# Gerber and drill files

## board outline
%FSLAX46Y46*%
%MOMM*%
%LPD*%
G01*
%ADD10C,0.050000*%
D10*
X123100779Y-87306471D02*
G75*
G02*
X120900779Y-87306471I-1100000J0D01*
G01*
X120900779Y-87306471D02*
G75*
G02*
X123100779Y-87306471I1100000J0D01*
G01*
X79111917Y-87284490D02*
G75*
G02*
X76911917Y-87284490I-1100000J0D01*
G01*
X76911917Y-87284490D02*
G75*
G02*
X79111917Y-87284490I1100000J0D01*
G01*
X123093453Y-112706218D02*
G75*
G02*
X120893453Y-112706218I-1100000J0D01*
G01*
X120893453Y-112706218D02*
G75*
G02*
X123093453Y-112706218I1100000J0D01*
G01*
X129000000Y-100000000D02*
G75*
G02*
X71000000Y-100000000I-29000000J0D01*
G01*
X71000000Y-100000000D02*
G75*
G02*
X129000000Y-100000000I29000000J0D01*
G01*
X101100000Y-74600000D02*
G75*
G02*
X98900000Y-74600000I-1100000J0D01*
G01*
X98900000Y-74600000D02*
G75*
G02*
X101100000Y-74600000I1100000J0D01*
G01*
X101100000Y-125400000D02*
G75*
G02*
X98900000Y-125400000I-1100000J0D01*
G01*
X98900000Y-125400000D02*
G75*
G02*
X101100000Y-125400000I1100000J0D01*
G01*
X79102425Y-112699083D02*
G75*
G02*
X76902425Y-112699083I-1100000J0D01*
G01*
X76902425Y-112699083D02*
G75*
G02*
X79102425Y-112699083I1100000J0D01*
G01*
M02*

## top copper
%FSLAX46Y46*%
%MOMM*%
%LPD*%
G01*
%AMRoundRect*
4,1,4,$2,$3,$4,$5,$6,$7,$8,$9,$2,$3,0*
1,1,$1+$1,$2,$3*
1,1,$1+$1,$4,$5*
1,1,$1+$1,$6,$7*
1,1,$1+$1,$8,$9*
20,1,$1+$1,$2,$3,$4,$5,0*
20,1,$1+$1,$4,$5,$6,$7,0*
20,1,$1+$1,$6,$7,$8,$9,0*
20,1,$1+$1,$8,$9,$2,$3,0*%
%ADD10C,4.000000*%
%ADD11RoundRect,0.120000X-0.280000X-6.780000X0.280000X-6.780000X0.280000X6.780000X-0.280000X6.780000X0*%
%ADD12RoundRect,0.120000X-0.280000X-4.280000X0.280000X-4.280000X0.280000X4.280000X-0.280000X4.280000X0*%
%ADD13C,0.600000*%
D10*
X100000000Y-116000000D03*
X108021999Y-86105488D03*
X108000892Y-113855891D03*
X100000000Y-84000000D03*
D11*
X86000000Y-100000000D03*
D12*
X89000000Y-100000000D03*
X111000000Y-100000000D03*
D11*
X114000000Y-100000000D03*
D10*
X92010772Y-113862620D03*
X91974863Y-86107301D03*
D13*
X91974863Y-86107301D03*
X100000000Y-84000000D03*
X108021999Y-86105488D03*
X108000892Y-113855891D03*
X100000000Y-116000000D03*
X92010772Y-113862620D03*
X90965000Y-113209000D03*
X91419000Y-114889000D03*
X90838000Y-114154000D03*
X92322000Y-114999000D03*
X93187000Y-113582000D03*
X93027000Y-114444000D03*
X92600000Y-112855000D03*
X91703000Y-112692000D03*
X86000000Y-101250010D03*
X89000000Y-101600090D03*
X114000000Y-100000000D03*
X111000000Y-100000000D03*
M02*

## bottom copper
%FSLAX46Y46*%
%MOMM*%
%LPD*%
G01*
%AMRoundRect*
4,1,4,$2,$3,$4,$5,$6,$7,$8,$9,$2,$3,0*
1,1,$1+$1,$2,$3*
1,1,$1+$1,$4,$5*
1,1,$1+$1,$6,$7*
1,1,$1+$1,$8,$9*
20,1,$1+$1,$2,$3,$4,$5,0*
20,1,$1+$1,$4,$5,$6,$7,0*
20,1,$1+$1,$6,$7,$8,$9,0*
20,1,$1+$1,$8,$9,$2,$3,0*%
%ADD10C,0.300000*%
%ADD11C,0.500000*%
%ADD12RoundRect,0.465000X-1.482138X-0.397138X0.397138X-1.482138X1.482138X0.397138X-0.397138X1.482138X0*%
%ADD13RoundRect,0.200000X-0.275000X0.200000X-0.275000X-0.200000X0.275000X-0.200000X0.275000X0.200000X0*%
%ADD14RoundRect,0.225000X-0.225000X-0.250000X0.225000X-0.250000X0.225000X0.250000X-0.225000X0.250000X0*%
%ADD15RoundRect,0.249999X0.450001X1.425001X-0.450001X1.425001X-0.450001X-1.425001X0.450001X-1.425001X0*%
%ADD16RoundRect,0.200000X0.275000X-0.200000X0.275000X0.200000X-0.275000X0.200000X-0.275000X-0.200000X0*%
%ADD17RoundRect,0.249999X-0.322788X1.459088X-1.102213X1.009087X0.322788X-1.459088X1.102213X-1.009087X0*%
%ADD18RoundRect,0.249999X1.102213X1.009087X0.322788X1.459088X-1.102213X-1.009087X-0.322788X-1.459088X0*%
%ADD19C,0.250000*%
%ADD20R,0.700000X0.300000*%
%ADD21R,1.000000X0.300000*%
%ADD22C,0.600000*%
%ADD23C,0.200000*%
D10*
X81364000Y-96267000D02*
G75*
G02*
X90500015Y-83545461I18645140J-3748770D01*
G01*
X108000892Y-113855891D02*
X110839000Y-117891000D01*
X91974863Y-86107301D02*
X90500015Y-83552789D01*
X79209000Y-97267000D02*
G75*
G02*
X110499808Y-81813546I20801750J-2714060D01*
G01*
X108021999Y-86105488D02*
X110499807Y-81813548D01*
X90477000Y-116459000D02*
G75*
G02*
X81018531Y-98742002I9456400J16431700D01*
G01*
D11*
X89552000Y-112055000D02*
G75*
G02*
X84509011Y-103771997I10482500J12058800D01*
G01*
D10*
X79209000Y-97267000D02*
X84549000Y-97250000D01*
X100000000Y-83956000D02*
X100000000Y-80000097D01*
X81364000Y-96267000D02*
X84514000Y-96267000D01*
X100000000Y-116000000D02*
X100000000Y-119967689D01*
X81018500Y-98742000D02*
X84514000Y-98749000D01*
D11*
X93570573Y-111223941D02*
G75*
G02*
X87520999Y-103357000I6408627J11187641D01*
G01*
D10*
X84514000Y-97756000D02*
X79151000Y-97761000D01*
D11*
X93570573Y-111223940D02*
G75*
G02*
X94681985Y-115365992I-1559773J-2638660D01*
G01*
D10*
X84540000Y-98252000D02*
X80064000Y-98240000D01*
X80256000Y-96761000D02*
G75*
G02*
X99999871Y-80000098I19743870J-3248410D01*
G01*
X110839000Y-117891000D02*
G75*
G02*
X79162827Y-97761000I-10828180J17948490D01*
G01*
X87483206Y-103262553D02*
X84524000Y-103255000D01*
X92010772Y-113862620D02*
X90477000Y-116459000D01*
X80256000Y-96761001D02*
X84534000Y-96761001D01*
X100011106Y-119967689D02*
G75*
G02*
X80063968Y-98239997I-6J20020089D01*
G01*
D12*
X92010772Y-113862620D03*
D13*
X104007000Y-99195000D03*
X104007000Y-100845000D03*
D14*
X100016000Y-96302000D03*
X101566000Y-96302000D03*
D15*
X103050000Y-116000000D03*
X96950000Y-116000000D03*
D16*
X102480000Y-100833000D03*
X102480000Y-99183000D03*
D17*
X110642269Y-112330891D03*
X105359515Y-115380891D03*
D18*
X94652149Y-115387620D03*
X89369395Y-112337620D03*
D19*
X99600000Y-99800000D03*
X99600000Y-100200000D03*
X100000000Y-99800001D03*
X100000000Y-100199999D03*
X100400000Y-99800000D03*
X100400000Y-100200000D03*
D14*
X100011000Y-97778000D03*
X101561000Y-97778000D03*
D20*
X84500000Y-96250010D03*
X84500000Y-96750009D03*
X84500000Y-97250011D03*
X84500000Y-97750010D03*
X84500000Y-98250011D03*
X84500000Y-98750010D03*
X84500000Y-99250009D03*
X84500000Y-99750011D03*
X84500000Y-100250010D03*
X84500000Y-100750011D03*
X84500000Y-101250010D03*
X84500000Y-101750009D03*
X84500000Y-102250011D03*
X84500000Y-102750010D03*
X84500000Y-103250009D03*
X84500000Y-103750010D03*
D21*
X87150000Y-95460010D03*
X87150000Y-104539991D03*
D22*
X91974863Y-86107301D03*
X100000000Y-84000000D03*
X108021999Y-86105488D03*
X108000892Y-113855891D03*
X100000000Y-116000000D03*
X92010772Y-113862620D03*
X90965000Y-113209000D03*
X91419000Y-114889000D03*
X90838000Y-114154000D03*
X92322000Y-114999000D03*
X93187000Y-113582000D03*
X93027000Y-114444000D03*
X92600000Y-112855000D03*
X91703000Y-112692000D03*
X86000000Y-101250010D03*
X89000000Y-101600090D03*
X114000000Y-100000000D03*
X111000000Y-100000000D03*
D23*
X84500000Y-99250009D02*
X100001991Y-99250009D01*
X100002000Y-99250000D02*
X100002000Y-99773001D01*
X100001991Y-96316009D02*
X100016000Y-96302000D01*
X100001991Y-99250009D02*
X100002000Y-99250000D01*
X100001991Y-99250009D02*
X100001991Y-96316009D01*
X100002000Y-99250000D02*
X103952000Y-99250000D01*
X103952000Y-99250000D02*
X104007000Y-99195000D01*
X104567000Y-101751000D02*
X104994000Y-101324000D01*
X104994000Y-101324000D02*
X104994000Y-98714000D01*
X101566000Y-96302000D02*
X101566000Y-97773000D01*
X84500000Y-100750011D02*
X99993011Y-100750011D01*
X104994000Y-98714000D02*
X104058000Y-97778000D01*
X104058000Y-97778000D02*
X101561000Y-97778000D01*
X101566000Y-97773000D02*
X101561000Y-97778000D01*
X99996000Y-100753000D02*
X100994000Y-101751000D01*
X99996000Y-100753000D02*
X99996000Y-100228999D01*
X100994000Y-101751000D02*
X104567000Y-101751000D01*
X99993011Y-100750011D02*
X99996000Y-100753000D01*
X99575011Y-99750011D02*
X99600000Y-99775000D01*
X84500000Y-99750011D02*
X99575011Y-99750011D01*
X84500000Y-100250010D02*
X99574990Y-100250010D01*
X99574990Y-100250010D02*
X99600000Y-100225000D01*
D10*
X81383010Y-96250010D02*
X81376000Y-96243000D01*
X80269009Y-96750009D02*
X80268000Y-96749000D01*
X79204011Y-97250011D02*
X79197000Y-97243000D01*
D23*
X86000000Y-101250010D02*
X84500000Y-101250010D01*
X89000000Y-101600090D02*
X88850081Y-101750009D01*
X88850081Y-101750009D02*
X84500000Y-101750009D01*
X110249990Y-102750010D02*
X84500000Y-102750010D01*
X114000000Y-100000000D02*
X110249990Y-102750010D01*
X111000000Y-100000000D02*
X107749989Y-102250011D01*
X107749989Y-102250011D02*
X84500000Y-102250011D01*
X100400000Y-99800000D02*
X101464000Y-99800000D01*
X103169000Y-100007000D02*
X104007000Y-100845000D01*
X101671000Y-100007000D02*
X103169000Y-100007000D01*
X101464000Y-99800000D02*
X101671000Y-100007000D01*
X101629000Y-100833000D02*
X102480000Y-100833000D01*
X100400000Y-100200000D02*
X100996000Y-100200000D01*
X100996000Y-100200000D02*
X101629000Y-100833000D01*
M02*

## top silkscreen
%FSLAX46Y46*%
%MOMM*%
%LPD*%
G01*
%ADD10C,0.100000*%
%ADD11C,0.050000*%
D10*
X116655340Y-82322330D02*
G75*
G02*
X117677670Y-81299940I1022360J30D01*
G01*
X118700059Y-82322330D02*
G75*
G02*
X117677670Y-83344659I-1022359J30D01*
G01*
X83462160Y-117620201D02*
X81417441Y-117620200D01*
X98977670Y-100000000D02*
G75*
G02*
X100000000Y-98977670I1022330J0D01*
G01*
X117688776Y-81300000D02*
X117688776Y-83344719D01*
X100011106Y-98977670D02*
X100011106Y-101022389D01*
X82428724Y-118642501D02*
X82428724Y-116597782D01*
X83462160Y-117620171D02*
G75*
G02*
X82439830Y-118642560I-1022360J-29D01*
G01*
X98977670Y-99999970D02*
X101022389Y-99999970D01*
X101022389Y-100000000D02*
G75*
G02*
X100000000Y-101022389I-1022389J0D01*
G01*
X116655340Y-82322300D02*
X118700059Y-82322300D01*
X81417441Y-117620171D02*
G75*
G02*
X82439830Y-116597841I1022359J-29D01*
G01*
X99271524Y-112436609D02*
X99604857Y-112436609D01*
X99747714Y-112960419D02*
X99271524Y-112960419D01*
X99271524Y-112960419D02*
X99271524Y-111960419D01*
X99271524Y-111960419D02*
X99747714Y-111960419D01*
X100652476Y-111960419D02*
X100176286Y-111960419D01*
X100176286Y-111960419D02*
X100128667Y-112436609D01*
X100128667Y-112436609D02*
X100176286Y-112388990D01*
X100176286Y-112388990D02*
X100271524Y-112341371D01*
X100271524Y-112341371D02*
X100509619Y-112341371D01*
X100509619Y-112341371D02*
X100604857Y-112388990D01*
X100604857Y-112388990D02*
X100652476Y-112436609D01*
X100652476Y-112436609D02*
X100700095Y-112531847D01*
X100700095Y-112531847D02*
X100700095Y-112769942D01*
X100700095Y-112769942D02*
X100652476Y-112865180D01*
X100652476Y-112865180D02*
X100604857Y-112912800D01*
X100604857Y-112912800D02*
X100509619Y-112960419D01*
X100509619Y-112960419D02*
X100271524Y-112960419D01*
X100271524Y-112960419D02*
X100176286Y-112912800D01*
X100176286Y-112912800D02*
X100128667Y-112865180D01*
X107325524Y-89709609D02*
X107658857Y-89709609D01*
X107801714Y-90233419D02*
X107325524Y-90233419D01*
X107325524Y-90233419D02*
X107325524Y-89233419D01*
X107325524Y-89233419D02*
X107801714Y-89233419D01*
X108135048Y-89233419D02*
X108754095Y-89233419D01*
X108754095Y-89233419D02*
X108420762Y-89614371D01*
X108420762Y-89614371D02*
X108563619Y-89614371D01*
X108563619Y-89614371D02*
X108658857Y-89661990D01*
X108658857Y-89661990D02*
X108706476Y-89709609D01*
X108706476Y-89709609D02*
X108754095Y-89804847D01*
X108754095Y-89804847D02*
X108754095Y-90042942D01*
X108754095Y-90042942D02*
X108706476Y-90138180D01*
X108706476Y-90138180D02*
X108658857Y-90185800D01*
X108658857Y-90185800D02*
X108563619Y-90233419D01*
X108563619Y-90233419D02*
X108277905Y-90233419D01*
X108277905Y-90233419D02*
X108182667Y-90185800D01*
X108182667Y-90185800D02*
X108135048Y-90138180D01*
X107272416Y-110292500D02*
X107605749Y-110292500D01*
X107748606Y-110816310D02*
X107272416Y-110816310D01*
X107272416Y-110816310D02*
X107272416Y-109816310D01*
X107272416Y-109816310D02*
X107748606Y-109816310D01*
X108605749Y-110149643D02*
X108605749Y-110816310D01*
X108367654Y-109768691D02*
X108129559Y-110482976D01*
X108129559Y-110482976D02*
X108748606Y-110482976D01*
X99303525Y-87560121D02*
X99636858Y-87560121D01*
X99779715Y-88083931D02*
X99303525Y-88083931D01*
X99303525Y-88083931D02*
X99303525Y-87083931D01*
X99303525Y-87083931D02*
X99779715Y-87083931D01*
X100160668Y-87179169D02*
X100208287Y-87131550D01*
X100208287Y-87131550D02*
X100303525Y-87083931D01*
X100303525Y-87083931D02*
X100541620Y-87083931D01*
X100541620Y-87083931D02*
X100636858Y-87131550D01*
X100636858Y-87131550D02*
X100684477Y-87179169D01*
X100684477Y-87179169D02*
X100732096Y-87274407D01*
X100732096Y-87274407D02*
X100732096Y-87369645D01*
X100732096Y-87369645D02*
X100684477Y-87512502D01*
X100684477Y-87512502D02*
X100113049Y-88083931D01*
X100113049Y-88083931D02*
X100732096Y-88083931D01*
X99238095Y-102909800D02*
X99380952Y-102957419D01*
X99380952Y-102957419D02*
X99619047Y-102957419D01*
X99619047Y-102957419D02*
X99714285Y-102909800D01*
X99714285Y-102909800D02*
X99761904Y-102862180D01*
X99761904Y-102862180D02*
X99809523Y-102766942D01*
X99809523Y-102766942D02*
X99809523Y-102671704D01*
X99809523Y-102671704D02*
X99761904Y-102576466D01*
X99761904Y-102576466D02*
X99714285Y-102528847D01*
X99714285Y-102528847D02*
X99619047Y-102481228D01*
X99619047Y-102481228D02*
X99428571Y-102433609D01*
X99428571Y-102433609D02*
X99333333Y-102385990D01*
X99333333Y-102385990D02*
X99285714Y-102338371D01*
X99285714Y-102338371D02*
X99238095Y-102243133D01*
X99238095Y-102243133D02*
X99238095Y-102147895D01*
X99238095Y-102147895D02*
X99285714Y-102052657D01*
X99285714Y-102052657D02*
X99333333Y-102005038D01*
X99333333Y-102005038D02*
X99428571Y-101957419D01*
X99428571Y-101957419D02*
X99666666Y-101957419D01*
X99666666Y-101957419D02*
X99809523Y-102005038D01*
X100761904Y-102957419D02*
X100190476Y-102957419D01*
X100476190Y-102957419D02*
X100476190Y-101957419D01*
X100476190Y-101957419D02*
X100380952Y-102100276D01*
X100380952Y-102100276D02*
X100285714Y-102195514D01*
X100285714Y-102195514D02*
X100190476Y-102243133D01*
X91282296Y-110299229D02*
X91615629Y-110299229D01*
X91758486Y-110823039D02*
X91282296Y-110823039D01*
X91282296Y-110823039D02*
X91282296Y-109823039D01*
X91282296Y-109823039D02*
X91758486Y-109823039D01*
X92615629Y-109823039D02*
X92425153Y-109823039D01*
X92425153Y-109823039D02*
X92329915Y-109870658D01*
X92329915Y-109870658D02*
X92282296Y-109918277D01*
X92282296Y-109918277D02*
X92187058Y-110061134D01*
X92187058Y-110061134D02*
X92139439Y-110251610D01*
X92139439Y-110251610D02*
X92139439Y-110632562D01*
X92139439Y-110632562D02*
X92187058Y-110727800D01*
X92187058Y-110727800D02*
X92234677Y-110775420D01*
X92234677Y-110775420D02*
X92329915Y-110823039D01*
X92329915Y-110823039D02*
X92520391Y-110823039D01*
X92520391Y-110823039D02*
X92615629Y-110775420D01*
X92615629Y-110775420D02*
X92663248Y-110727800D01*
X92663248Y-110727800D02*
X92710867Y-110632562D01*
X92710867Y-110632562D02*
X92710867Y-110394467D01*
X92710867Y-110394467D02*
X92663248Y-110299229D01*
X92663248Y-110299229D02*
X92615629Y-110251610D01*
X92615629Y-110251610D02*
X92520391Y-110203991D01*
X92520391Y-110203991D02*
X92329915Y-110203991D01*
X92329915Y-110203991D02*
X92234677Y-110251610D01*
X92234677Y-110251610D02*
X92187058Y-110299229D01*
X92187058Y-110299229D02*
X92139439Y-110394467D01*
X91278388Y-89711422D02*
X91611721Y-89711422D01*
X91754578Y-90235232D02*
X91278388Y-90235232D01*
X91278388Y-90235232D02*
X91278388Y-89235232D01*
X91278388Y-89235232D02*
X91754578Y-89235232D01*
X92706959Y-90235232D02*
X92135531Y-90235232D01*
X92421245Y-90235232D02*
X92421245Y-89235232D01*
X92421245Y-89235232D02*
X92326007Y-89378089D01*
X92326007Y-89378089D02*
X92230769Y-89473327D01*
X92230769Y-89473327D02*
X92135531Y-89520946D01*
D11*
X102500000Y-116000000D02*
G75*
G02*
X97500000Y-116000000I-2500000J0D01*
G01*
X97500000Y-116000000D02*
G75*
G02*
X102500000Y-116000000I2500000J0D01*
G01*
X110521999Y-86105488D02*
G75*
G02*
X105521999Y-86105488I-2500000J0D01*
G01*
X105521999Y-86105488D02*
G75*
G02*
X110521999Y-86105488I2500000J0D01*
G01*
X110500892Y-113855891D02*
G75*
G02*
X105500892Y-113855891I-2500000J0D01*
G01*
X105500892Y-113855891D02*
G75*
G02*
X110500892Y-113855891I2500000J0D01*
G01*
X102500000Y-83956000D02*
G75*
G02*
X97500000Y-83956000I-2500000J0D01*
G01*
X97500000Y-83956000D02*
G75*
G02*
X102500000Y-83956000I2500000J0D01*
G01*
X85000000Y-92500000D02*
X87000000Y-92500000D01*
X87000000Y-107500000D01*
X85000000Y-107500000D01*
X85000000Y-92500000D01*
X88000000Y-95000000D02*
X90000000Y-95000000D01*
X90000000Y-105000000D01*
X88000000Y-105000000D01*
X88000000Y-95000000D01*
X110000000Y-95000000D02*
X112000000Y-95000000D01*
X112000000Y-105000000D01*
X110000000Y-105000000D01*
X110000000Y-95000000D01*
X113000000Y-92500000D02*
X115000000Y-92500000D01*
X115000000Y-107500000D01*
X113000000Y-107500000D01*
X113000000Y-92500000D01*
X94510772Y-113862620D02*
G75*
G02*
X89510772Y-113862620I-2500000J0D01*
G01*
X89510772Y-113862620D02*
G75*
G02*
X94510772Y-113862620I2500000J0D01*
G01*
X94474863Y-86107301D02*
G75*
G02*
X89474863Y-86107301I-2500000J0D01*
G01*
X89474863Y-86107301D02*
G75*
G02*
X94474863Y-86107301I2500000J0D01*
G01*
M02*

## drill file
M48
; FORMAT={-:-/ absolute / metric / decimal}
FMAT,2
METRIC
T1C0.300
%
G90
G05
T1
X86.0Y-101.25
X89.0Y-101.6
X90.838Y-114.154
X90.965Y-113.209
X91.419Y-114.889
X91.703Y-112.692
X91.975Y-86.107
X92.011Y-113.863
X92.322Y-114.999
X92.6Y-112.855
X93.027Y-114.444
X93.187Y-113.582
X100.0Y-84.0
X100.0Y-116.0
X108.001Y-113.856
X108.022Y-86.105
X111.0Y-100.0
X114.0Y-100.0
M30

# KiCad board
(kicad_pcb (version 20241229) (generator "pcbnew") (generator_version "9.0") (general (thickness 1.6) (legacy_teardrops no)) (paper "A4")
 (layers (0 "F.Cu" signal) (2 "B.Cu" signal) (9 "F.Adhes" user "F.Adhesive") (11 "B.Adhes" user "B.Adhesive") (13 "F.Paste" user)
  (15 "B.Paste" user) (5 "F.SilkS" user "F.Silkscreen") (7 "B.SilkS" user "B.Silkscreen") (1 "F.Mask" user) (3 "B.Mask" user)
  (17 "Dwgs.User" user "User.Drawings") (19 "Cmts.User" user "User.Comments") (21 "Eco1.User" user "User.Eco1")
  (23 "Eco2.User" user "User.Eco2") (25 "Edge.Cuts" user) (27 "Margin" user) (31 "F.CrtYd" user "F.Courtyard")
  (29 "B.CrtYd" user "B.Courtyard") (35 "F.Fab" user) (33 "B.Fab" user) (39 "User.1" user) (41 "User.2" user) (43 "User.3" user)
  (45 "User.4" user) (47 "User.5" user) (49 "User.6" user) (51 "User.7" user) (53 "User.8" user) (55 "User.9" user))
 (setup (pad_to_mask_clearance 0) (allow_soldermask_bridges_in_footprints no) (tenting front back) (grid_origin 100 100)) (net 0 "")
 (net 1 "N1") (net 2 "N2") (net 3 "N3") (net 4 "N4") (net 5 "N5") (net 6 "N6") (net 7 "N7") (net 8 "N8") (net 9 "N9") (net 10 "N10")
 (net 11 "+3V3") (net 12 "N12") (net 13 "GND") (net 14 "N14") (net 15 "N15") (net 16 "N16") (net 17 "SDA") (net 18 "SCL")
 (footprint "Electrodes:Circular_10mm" (layer "F.Cu") (at 100 116)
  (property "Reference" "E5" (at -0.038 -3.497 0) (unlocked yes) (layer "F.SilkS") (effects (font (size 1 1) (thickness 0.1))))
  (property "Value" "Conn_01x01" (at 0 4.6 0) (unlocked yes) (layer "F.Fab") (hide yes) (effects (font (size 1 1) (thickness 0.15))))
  (fp_circle (center 0 0) (end 2.5 0) (stroke (width 0.05) (type solid)) (fill no) (layer "F.SilkS"))
  (pad "1" smd circle (at 0 0) (size 4 4) (layers "F.Cu" "F.Mask" "F.Paste") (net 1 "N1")))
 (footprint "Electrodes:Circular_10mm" (layer "F.Cu") (at 108.021999 86.105488)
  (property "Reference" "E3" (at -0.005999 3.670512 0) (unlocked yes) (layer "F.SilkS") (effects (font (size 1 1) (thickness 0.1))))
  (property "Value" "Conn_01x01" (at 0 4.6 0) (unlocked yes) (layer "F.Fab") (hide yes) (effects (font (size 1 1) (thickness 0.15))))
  (fp_circle (center 0 0) (end 2.5 0) (stroke (width 0.05) (type solid)) (fill no) (layer "F.SilkS"))
  (pad "1" smd circle (at 0 0) (size 4 4) (layers "F.Cu" "F.Mask" "F.Paste") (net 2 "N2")))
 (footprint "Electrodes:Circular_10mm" (layer "F.Cu") (at 108.000892 113.855891)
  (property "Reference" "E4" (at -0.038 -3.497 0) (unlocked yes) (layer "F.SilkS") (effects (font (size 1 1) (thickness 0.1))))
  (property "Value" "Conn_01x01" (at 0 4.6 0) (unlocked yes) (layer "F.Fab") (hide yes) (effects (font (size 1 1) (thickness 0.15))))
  (fp_circle (center 0 0) (end 2.5 0) (stroke (width 0.05) (type solid)) (fill no) (layer "F.SilkS"))
  (pad "1" smd circle (at 0 0) (size 4 4) (layers "F.Cu" "F.Mask" "F.Paste") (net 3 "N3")))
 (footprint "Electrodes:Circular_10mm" (layer "F.Cu") (at 100 83.956)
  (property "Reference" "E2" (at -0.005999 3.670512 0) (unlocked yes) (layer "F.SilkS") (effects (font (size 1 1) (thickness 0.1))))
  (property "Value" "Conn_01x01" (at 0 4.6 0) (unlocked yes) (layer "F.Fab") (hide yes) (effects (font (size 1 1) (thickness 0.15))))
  (fp_circle (center 0 0) (end 2.5 0) (stroke (width 0.05) (type solid)) (fill no) (layer "F.SilkS"))
  (pad "1" smd circle (at 0 0.044) (size 4 4) (layers "F.Cu" "F.Mask" "F.Paste") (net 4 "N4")))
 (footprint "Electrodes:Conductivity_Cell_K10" (layer "F.Cu") (at 100 100)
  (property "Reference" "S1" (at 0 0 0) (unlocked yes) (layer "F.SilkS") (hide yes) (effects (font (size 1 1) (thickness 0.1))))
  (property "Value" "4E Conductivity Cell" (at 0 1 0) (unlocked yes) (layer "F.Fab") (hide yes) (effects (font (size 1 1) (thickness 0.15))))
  (fp_rect (start -15 -7.5) (end -13 7.5) (stroke (width 0.05) (type solid)) (fill no) (layer "F.SilkS"))
  (fp_rect (start -12 -5) (end -10 5) (stroke (width 0.05) (type solid)) (fill no) (layer "F.SilkS"))
  (fp_rect (start 10 -5) (end 12 5) (stroke (width 0.05) (type solid)) (fill no) (layer "F.SilkS"))
  (fp_rect (start 13 -7.5) (end 15 7.5) (stroke (width 0.05) (type solid)) (fill no) (layer "F.SilkS"))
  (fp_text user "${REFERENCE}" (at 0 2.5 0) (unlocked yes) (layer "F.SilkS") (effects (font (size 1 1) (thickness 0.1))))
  (pad "1" smd roundrect (at -14 0) (size 0.8 13.8) (layers "F.Cu" "F.Mask" "F.Paste") (roundrect_rratio 0.15) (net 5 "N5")
   (thermal_bridge_angle 45))
  (pad "2" smd roundrect (at -11 0) (size 0.8 8.8) (layers "F.Cu" "F.Mask" "F.Paste") (roundrect_rratio 0.15) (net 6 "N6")
   (thermal_bridge_angle 45))
  (pad "3" smd roundrect (at 11 0) (size 0.8 8.8) (layers "F.Cu" "F.Mask" "F.Paste") (roundrect_rratio 0.15) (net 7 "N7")
   (thermal_bridge_angle 45))
  (pad "4" smd roundrect (at 14 0) (size 0.8 13.8) (layers "F.Cu" "F.Mask" "F.Paste") (roundrect_rratio 0.15) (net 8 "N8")
   (thermal_bridge_angle 45)))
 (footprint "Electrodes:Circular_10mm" (layer "F.Cu") (at 92.010772 113.86262)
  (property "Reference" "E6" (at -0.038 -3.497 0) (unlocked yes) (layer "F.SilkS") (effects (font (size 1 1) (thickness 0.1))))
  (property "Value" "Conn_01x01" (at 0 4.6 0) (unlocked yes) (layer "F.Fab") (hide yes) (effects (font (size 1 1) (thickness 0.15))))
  (fp_circle (center 0 0) (end 2.5 0) (stroke (width 0.05) (type solid)) (fill no) (layer "F.SilkS"))
  (pad "1" smd circle (at 0 0) (size 4 4) (layers "F.Cu" "F.Mask" "F.Paste") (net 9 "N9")))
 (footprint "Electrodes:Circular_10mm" (layer "F.Cu") (at 91.974863 86.107301)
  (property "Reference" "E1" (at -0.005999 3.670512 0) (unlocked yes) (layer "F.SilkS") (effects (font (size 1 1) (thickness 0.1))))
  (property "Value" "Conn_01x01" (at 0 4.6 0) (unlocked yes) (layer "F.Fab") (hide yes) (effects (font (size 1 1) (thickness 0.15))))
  (fp_circle (center 0 0) (end 2.5 0) (stroke (width 0.05) (type solid)) (fill no) (layer "F.SilkS"))
  (pad "1" smd circle (at 0 0) (size 4 4) (layers "F.Cu" "F.Mask" "F.Paste") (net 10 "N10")))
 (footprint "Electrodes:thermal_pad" (layer "B.Cu") (at 92.010772 113.86262)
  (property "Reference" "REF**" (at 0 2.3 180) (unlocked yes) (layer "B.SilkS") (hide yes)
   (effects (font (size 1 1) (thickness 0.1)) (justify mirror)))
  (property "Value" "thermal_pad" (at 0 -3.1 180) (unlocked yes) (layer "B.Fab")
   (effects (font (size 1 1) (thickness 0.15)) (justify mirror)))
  (pad "1" smd roundrect (at 0 0 330) (size 3.1 3.1) (layers "B.Cu" "B.Mask" "B.Paste") (roundrect_rratio 0.15) (thermal_bridge_angle 45)))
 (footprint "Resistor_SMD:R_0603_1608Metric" (layer "B.Cu") (at 104.007 100.02 -90)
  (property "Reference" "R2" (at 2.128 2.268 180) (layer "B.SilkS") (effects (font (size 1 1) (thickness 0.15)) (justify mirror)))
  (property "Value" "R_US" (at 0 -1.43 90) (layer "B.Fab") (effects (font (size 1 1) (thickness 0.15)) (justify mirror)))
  (pad "1" smd roundrect (at -0.825 0 270) (size 0.8 0.95) (layers "B.Cu" "B.Mask" "B.Paste") (roundrect_rratio 0.25) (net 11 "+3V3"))
  (pad "2" smd roundrect (at 0.825 0 270) (size 0.8 0.95) (layers "B.Cu" "B.Mask" "B.Paste") (roundrect_rratio 0.25) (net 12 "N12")))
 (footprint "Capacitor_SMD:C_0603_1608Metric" (layer "B.Cu") (at 100.791 96.302)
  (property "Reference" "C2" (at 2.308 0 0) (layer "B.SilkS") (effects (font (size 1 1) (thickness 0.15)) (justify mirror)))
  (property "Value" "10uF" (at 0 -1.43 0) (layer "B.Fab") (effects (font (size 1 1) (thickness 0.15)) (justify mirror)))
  (pad "1" smd roundrect (at -0.775 0) (size 0.9 0.95) (layers "B.Cu" "B.Mask" "B.Paste") (roundrect_rratio 0.25) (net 11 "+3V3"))
  (pad "2" smd roundrect (at 0.775 0) (size 0.9 0.95) (layers "B.Cu" "B.Mask" "B.Paste") (roundrect_rratio 0.25) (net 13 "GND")))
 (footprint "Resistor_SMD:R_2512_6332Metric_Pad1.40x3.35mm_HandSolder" (layer "B.Cu") (at 100 116 180)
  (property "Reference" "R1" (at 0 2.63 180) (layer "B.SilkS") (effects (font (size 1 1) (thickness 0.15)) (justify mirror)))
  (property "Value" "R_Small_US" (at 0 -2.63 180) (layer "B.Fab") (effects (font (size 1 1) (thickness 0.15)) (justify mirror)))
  (pad "1" smd roundrect (at -3.05 0 180) (size 1.4 3.35) (layers "B.Cu" "B.Mask" "B.Paste") (roundrect_rratio 0.178571))
  (pad "2" smd roundrect (at 3.05 0 180) (size 1.4 3.35) (layers "B.Cu" "B.Mask" "B.Paste") (roundrect_rratio 0.178571)))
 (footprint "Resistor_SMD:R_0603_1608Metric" (layer "B.Cu") (at 102.48 100.008 90)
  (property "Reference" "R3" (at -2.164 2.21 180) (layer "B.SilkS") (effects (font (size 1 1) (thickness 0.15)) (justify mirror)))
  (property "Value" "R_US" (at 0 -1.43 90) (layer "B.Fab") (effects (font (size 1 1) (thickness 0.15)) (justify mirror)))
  (pad "1" smd roundrect (at -0.825 0 90) (size 0.8 0.95) (layers "B.Cu" "B.Mask" "B.Paste") (roundrect_rratio 0.25) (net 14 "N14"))
  (pad "2" smd roundrect (at 0.825 0 90) (size 0.8 0.95) (layers "B.Cu" "B.Mask" "B.Paste") (roundrect_rratio 0.25) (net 11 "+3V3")))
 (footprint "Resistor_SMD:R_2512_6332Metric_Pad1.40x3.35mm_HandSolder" (layer "B.Cu") (at 108.000892 113.855891 -150)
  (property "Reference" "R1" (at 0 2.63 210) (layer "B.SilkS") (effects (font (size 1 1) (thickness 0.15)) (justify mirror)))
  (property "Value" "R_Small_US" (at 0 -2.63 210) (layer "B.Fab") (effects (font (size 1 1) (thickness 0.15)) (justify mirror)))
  (pad "1" smd roundrect (at -3.05 0 210) (size 1.4 3.35) (layers "B.Cu" "B.Mask" "B.Paste") (roundrect_rratio 0.178571))
  (pad "2" smd roundrect (at 3.05 0 210) (size 1.4 3.35) (layers "B.Cu" "B.Mask" "B.Paste") (roundrect_rratio 0.178571)))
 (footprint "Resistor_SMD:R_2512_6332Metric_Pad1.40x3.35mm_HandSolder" (layer "B.Cu") (at 92.010772 113.86262 150)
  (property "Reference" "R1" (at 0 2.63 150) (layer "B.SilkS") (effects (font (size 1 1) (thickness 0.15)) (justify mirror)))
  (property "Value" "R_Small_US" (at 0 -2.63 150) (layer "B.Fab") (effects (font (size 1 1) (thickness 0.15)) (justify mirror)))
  (pad "1" smd roundrect (at -3.05 0 150) (size 1.4 3.35) (layers "B.Cu" "B.Mask" "B.Paste") (roundrect_rratio 0.178571) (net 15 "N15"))
  (pad "2" smd roundrect (at 3.05 0 150) (size 1.4 3.35) (layers "B.Cu" "B.Mask" "B.Paste") (roundrect_rratio 0.178571) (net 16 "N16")))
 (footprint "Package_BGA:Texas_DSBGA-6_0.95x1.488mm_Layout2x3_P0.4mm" (layer "B.Cu") (at 100 100 -90)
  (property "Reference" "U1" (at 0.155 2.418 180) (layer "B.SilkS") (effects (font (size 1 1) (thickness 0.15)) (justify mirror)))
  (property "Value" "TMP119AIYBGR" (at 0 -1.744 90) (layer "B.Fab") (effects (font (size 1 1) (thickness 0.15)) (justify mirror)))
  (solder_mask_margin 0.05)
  (pad "A1" smd circle (at -0.2 0.4 270) (size 0.25 0.25) (layers "B.Cu" "B.Mask" "B.Paste") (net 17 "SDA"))
  (pad "A2" smd circle (at 0.2 0.4 270) (size 0.25 0.25) (layers "B.Cu" "B.Mask" "B.Paste") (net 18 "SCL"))
  (pad "B1" smd circle (at -0.199999 0 270) (size 0.25 0.25) (layers "B.Cu" "B.Mask" "B.Paste") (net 11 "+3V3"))
  (pad "B2" smd circle (at 0.199999 0 270) (size 0.25 0.25) (layers "B.Cu" "B.Mask" "B.Paste") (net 13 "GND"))
  (pad "C1" smd circle (at -0.2 -0.4 270) (size 0.25 0.25) (layers "B.Cu" "B.Mask" "B.Paste") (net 12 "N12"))
  (pad "C2" smd circle (at 0.2 -0.4 270) (size 0.25 0.25) (layers "B.Cu" "B.Mask" "B.Paste") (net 14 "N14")))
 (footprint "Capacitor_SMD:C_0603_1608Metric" (layer "B.Cu") (at 100.786 97.778)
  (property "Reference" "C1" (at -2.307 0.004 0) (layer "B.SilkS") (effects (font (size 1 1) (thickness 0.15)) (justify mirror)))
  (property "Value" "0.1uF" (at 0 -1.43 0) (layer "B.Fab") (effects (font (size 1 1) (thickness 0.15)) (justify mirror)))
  (pad "1" smd roundrect (at -0.775 0) (size 0.9 0.95) (layers "B.Cu" "B.Mask" "B.Paste") (roundrect_rratio 0.25) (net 11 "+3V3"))
  (pad "2" smd roundrect (at 0.775 0) (size 0.9 0.95) (layers "B.Cu" "B.Mask" "B.Paste") (roundrect_rratio 0.25) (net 13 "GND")))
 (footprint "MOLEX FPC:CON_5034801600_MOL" (layer "B.Cu") (at 86 100 -90)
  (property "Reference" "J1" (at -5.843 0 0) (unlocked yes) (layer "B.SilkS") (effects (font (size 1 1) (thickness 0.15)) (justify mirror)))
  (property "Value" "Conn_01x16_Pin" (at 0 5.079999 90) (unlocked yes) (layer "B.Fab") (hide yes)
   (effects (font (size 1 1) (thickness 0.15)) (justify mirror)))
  (pad "1" smd rect (at -3.74999 1.5 270) (size 0.3 0.7) (layers "B.Cu" "B.Mask" "B.Paste") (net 10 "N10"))
  (pad "2" smd rect (at -3.249991 1.5 270) (size 0.3 0.7) (layers "B.Cu" "B.Mask" "B.Paste") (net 4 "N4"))
  (pad "3" smd rect (at -2.749989 1.5 270) (size 0.3 0.7) (layers "B.Cu" "B.Mask" "B.Paste") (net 2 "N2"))
  (pad "4" smd rect (at -2.24999 1.5 270) (size 0.3 0.7) (layers "B.Cu" "B.Mask" "B.Paste") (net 3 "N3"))
  (pad "5" smd rect (at -1.749989 1.5 270) (size 0.3 0.7) (layers "B.Cu" "B.Mask" "B.Paste") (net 1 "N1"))
  (pad "6" smd rect (at -1.24999 1.5 270) (size 0.3 0.7) (layers "B.Cu" "B.Mask" "B.Paste") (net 9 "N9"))
  (pad "7" smd rect (at -0.749991 1.5 270) (size 0.3 0.7) (layers "B.Cu" "B.Mask" "B.Paste") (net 11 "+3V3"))
  (pad "8" smd rect (at -0.249989 1.5 270) (size 0.3 0.7) (layers "B.Cu" "B.Mask" "B.Paste") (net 17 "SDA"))
  (pad "9" smd rect (at 0.25001 1.5 270) (size 0.3 0.7) (layers "B.Cu" "B.Mask" "B.Paste") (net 18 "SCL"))
  (pad "10" smd rect (at 0.750011 1.5 270) (size 0.3 0.7) (layers "B.Cu" "B.Mask" "B.Paste") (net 13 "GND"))
  (pad "11" smd rect (at 1.25001 1.5 270) (size 0.3 0.7) (layers "B.Cu" "B.Mask" "B.Paste") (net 5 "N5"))
  (pad "12" smd rect (at 1.750009 1.5 270) (size 0.3 0.7) (layers "B.Cu" "B.Mask" "B.Paste") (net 6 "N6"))
  (pad "13" smd rect (at 2.250011 1.5 270) (size 0.3 0.7) (layers "B.Cu" "B.Mask" "B.Paste") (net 7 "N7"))
  (pad "14" smd rect (at 2.75001 1.5 270) (size 0.3 0.7) (layers "B.Cu" "B.Mask" "B.Paste") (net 8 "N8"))
  (pad "15" smd rect (at 3.250009 1.5 270) (size 0.3 0.7) (layers "B.Cu" "B.Mask" "B.Paste") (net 15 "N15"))
  (pad "16" smd rect (at 3.75001 1.5 270) (size 0.3 0.7) (layers "B.Cu" "B.Mask" "B.Paste") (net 16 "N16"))
  (pad "P1" smd rect (at -4.53999 -1.15 270) (size 0.3 1) (layers "B.Cu" "B.Mask" "B.Paste"))
  (pad "P2" smd rect (at 4.539991 -1.15 270) (size 0.3 1) (layers "B.Cu" "B.Mask" "B.Paste")))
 (gr_arc (start 81.364 96.267) (mid 84.561647 88.922101) (end 90.500015 83.545461) (stroke (width 0.3) (type solid)) (layer "B.Cu") (net 10))
 (gr_line (start 108.000892 113.855891) (end 110.839 117.891) (stroke (width 0.3) (type default)) (layer "B.Cu") (net 3))
 (gr_line (start 91.974863 86.107301) (end 90.500015 83.552789) (stroke (width 0.3) (type solid)) (layer "B.Cu") (net 10))
 (gr_arc (start 79.209 97.267) (mid 90.721498 81.171791) (end 110.499807 81.813548) (stroke (width 0.3) (type solid)) (layer "B.Cu") (net 2))
 (gr_line (start 108.021999 86.105488) (end 110.499807 81.813548) (stroke (width 0.3) (type default)) (layer "B.Cu") (net 2))
 (gr_arc (start 90.477 116.459) (mid 83.208992 108.955856) (end 81.0185 98.742) (stroke (width 0.3) (type solid)) (layer "B.Cu") (net 9))
 (gr_arc (start 89.552 112.055) (mid 86.386934 108.305327) (end 84.509 103.772) (stroke (width 0.5) (type default)) (layer "B.Cu") (net 16))
 (gr_line (start 79.209 97.267) (end 84.549 97.25) (stroke (width 0.3) (type default)) (layer "B.Cu") (net 2))
 (gr_line (start 100 83.956) (end 100 80.000097) (stroke (width 0.3) (type default)) (layer "B.Cu") (net 4))
 (gr_line (start 81.364 96.267) (end 84.514 96.267) (stroke (width 0.3) (type solid)) (layer "B.Cu") (net 10))
 (gr_line (start 100 116) (end 100 119.967689) (stroke (width 0.3) (type default)) (layer "B.Cu") (net 1))
 (gr_line (start 81.0185 98.742) (end 84.514 98.749) (stroke (width 0.3) (type default)) (layer "B.Cu") (net 9))
 (gr_arc (start 93.570573 111.223941) (mid 89.758558 107.895839) (end 87.521 103.357) (stroke (width 0.5) (type default)) (layer "B.Cu")
  (net 15))
 (gr_line (start 84.514 97.756) (end 79.151 97.761) (stroke (width 0.3) (type default)) (layer "B.Cu") (net 3))
 (gr_arc (start 93.570573 111.22394) (mid 94.971273 113.068237) (end 94.682 115.366) (stroke (width 0.5) (type default)) (layer "B.Cu")
  (net 15))
 (gr_line (start 84.54 98.252) (end 80.064 98.24) (stroke (width 0.3) (type default)) (layer "B.Cu") (net 1))
 (gr_arc (start 80.256 96.761) (mid 87.050466 84.755377) (end 99.999871 80.000097) (stroke (width 0.3) (type solid)) (layer "B.Cu") (net 4))
 (gr_arc (start 110.839 117.891) (mid 88.767893 117.634157) (end 79.162823 97.761) (stroke (width 0.3) (type default)) (layer "B.Cu")
  (net 3))
 (gr_line (start 87.483206 103.262553) (end 84.524 103.255) (stroke (width 0.3) (type default)) (layer "B.Cu") (net 15))
 (gr_line (start 92.010772 113.86262) (end 90.477 116.459) (stroke (width 0.3) (type default)) (layer "B.Cu") (net 9))
 (gr_line (start 80.256 96.761001) (end 84.534 96.761001) (stroke (width 0.3) (type default)) (layer "B.Cu") (net 4))
 (gr_arc (start 100.011106 119.967689) (mid 85.263398 113.486757) (end 80.064 98.24) (stroke (width 0.3) (type default)) (layer "B.Cu")
  (net 1))
 (gr_arc (start 116.65534 82.32233) (mid 116.954774 81.599434) (end 117.67767 81.3) (stroke (width 0.1) (type default)) (layer "F.SilkS"))
 (gr_arc (start 118.700059 82.32233) (mid 118.400608 83.045268) (end 117.67767 83.344719) (stroke (width 0.1) (type default))
  (layer "F.SilkS"))
 (gr_line (start 83.46216 117.620201) (end 81.417441 117.6202) (stroke (width 0.1) (type default)) (layer "F.SilkS"))
 (gr_arc (start 98.97767 100) (mid 99.277104 99.277104) (end 100 98.97767) (stroke (width 0.1) (type default)) (layer "F.SilkS"))
 (gr_line (start 117.688776 81.3) (end 117.688776 83.344719) (stroke (width 0.1) (type default)) (layer "F.SilkS"))
 (gr_line (start 100.011106 98.97767) (end 100.011106 101.022389) (stroke (width 0.1) (type default)) (layer "F.SilkS"))
 (gr_line (start 82.428724 118.642501) (end 82.428724 116.597782) (stroke (width 0.1) (type default)) (layer "F.SilkS"))
 (gr_arc (start 83.46216 117.620171) (mid 83.162726 118.343067) (end 82.43983 118.642501) (stroke (width 0.1) (type default))
  (layer "F.SilkS"))
 (gr_line (start 98.97767 99.99997) (end 101.022389 99.99997) (stroke (width 0.1) (type default)) (layer "F.SilkS"))
 (gr_arc (start 101.022389 100) (mid 100.722938 100.722938) (end 100 101.022389) (stroke (width 0.1) (type default)) (layer "F.SilkS"))
 (gr_line (start 116.65534 82.3223) (end 118.700059 82.3223) (stroke (width 0.1) (type default)) (layer "F.SilkS"))
 (gr_arc (start 81.417441 117.620171) (mid 81.716892 116.897233) (end 82.43983 116.597782) (stroke (width 0.1) (type default))
  (layer "F.SilkS"))
 (gr_circle (center 122.000779 87.306471) (end 123.100779 87.306471) (stroke (width 0.05) (type default)) (fill no) (layer "Edge.Cuts"))
 (gr_circle (center 78.011917 87.28449) (end 79.111917 87.28449) (stroke (width 0.05) (type default)) (fill no) (layer "Edge.Cuts"))
 (gr_circle (center 121.993453 112.706218) (end 123.093453 112.706218) (stroke (width 0.05) (type default)) (fill no) (layer "Edge.Cuts"))
 (gr_circle (center 100 100) (end 129 100) (stroke (width 0.05) (type default)) (fill no) (layer "Edge.Cuts"))
 (gr_circle (center 100 74.6) (end 101.1 74.6) (stroke (width 0.05) (type default)) (fill no) (layer "Edge.Cuts"))
 (gr_circle (center 100 125.4) (end 101.1 125.4) (stroke (width 0.05) (type default)) (fill no) (layer "Edge.Cuts"))
 (gr_circle (center 78.002425 112.699083) (end 79.102425 112.699083) (stroke (width 0.05) (type default)) (fill no) (layer "Edge.Cuts"))
 (segment (start 84.5 99.250009) (end 100.001991 99.250009) (width 0.2) (layer "B.Cu") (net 11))
 (segment (start 100.002 99.25) (end 100.002 99.773001) (width 0.2) (layer "B.Cu") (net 11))
 (segment (start 100.001991 96.316009) (end 100.016 96.302) (width 0.2) (layer "B.Cu") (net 11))
 (segment (start 100.001991 99.250009) (end 100.002 99.25) (width 0.2) (layer "B.Cu") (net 11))
 (segment (start 100.001991 99.250009) (end 100.001991 96.316009) (width 0.2) (layer "B.Cu") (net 11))
 (segment (start 100.002 99.25) (end 103.952 99.25) (width 0.2) (layer "B.Cu") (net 11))
 (segment (start 103.952 99.25) (end 104.007 99.195) (width 0.2) (layer "B.Cu") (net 11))
 (segment (start 104.567 101.751) (end 104.994 101.324) (width 0.2) (layer "B.Cu") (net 13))
 (segment (start 104.994 101.324) (end 104.994 98.714) (width 0.2) (layer "B.Cu") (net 13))
 (segment (start 101.566 96.302) (end 101.566 97.773) (width 0.2) (layer "B.Cu") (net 13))
 (segment (start 84.5 100.750011) (end 99.993011 100.750011) (width 0.2) (layer "B.Cu") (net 13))
 (segment (start 104.994 98.714) (end 104.058 97.778) (width 0.2) (layer "B.Cu") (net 13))
 (segment (start 104.058 97.778) (end 101.561 97.778) (width 0.2) (layer "B.Cu") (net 13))
 (segment (start 101.566 97.773) (end 101.561 97.778) (width 0.2) (layer "B.Cu") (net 13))
 (segment (start 99.996 100.753) (end 100.994 101.751) (width 0.2) (layer "B.Cu") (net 13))
 (segment (start 99.996 100.753) (end 99.996 100.228999) (width 0.2) (layer "B.Cu") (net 13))
 (segment (start 100.994 101.751) (end 104.567 101.751) (width 0.2) (layer "B.Cu") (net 13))
 (segment (start 99.993011 100.750011) (end 99.996 100.753) (width 0.2) (layer "B.Cu") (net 13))
 (segment (start 99.575011 99.750011) (end 99.6 99.775) (width 0.2) (layer "B.Cu") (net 17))
 (segment (start 84.5 99.750011) (end 99.575011 99.750011) (width 0.2) (layer "B.Cu") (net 17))
 (segment (start 84.5 100.25001) (end 99.57499 100.25001) (width 0.2) (layer "B.Cu") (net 18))
 (segment (start 99.57499 100.25001) (end 99.6 100.225) (width 0.2) (layer "B.Cu") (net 18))
 (via (at 91.974863 86.107301) (size 0.6) (drill 0.3) (layers "F.Cu" "B.Cu") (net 10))
 (segment (start 81.38301 96.25001) (end 81.376 96.243) (width 0.3) (layer "B.Cu") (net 10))
 (via (at 100 84) (size 0.6) (drill 0.3) (layers "F.Cu" "B.Cu") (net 4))
 (segment (start 80.269009 96.750009) (end 80.268 96.749) (width 0.3) (layer "B.Cu") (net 4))
 (via (at 108.021999 86.105488) (size 0.6) (drill 0.3) (layers "F.Cu" "B.Cu") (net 2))
 (segment (start 79.204011 97.250011) (end 79.197 97.243) (width 0.3) (layer "B.Cu") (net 2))
 (via (at 108.000892 113.855891) (size 0.6) (drill 0.3) (layers "F.Cu" "B.Cu") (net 3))
 (via (at 100 116) (size 0.6) (drill 0.3) (layers "F.Cu" "B.Cu") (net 1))
 (via (at 92.010772 113.86262) (size 0.6) (drill 0.3) (layers "F.Cu" "B.Cu") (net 9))
 (via (at 90.965 113.209) (size 0.6) (drill 0.3) (layers "F.Cu" "B.Cu") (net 9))
 (via (at 91.419 114.889) (size 0.6) (drill 0.3) (layers "F.Cu" "B.Cu") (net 9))
 (via (at 90.838 114.154) (size 0.6) (drill 0.3) (layers "F.Cu" "B.Cu") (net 9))
 (via (at 92.322 114.999) (size 0.6) (drill 0.3) (layers "F.Cu" "B.Cu") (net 9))
 (via (at 93.187 113.582) (size 0.6) (drill 0.3) (layers "F.Cu" "B.Cu") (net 9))
 (via (at 93.027 114.444) (size 0.6) (drill 0.3) (layers "F.Cu" "B.Cu") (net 9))
 (via (at 92.6 112.855) (size 0.6) (drill 0.3) (layers "F.Cu" "B.Cu") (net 9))
 (via (at 91.703 112.692) (size 0.6) (drill 0.3) (layers "F.Cu" "B.Cu") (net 9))
 (via (at 86 101.25001) (size 0.6) (drill 0.3) (layers "F.Cu" "B.Cu") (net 5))
 (segment (start 86 101.25001) (end 84.5 101.25001) (width 0.2) (layer "B.Cu") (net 5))
 (via (at 89 101.60009) (size 0.6) (drill 0.3) (layers "F.Cu" "B.Cu") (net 6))
 (segment (start 89 101.60009) (end 88.850081 101.750009) (width 0.2) (layer "B.Cu") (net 6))
 (segment (start 88.850081 101.750009) (end 84.5 101.750009) (width 0.2) (layer "B.Cu") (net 6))
 (via (at 114 100) (size 0.6) (drill 0.3) (layers "F.Cu" "B.Cu") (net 8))
 (segment (start 110.24999 102.75001) (end 84.5 102.75001) (width 0.2) (layer "B.Cu") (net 8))
 (segment (start 114 100) (end 110.24999 102.75001) (width 0.2) (layer "B.Cu") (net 8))
 (via (at 111 100) (size 0.6) (drill 0.3) (layers "F.Cu" "B.Cu") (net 7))
 (segment (start 111 100) (end 107.749989 102.250011) (width 0.2) (layer "B.Cu") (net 7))
 (segment (start 107.749989 102.250011) (end 84.5 102.250011) (width 0.2) (layer "B.Cu") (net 7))
 (segment (start 100.4 99.8) (end 101.464 99.8) (width 0.2) (layer "B.Cu") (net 12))
 (segment (start 103.169 100.007) (end 104.007 100.845) (width 0.2) (layer "B.Cu") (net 12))
 (segment (start 101.671 100.007) (end 103.169 100.007) (width 0.2) (layer "B.Cu") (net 12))
 (segment (start 101.464 99.8) (end 101.671 100.007) (width 0.2) (layer "B.Cu") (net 12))
 (segment (start 101.629 100.833) (end 102.48 100.833) (width 0.2) (layer "B.Cu") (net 14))
 (segment (start 100.4 100.2) (end 100.996 100.2) (width 0.2) (layer "B.Cu") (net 14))
 (segment (start 100.996 100.2) (end 101.629 100.833) (width 0.2) (layer "B.Cu") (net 14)))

